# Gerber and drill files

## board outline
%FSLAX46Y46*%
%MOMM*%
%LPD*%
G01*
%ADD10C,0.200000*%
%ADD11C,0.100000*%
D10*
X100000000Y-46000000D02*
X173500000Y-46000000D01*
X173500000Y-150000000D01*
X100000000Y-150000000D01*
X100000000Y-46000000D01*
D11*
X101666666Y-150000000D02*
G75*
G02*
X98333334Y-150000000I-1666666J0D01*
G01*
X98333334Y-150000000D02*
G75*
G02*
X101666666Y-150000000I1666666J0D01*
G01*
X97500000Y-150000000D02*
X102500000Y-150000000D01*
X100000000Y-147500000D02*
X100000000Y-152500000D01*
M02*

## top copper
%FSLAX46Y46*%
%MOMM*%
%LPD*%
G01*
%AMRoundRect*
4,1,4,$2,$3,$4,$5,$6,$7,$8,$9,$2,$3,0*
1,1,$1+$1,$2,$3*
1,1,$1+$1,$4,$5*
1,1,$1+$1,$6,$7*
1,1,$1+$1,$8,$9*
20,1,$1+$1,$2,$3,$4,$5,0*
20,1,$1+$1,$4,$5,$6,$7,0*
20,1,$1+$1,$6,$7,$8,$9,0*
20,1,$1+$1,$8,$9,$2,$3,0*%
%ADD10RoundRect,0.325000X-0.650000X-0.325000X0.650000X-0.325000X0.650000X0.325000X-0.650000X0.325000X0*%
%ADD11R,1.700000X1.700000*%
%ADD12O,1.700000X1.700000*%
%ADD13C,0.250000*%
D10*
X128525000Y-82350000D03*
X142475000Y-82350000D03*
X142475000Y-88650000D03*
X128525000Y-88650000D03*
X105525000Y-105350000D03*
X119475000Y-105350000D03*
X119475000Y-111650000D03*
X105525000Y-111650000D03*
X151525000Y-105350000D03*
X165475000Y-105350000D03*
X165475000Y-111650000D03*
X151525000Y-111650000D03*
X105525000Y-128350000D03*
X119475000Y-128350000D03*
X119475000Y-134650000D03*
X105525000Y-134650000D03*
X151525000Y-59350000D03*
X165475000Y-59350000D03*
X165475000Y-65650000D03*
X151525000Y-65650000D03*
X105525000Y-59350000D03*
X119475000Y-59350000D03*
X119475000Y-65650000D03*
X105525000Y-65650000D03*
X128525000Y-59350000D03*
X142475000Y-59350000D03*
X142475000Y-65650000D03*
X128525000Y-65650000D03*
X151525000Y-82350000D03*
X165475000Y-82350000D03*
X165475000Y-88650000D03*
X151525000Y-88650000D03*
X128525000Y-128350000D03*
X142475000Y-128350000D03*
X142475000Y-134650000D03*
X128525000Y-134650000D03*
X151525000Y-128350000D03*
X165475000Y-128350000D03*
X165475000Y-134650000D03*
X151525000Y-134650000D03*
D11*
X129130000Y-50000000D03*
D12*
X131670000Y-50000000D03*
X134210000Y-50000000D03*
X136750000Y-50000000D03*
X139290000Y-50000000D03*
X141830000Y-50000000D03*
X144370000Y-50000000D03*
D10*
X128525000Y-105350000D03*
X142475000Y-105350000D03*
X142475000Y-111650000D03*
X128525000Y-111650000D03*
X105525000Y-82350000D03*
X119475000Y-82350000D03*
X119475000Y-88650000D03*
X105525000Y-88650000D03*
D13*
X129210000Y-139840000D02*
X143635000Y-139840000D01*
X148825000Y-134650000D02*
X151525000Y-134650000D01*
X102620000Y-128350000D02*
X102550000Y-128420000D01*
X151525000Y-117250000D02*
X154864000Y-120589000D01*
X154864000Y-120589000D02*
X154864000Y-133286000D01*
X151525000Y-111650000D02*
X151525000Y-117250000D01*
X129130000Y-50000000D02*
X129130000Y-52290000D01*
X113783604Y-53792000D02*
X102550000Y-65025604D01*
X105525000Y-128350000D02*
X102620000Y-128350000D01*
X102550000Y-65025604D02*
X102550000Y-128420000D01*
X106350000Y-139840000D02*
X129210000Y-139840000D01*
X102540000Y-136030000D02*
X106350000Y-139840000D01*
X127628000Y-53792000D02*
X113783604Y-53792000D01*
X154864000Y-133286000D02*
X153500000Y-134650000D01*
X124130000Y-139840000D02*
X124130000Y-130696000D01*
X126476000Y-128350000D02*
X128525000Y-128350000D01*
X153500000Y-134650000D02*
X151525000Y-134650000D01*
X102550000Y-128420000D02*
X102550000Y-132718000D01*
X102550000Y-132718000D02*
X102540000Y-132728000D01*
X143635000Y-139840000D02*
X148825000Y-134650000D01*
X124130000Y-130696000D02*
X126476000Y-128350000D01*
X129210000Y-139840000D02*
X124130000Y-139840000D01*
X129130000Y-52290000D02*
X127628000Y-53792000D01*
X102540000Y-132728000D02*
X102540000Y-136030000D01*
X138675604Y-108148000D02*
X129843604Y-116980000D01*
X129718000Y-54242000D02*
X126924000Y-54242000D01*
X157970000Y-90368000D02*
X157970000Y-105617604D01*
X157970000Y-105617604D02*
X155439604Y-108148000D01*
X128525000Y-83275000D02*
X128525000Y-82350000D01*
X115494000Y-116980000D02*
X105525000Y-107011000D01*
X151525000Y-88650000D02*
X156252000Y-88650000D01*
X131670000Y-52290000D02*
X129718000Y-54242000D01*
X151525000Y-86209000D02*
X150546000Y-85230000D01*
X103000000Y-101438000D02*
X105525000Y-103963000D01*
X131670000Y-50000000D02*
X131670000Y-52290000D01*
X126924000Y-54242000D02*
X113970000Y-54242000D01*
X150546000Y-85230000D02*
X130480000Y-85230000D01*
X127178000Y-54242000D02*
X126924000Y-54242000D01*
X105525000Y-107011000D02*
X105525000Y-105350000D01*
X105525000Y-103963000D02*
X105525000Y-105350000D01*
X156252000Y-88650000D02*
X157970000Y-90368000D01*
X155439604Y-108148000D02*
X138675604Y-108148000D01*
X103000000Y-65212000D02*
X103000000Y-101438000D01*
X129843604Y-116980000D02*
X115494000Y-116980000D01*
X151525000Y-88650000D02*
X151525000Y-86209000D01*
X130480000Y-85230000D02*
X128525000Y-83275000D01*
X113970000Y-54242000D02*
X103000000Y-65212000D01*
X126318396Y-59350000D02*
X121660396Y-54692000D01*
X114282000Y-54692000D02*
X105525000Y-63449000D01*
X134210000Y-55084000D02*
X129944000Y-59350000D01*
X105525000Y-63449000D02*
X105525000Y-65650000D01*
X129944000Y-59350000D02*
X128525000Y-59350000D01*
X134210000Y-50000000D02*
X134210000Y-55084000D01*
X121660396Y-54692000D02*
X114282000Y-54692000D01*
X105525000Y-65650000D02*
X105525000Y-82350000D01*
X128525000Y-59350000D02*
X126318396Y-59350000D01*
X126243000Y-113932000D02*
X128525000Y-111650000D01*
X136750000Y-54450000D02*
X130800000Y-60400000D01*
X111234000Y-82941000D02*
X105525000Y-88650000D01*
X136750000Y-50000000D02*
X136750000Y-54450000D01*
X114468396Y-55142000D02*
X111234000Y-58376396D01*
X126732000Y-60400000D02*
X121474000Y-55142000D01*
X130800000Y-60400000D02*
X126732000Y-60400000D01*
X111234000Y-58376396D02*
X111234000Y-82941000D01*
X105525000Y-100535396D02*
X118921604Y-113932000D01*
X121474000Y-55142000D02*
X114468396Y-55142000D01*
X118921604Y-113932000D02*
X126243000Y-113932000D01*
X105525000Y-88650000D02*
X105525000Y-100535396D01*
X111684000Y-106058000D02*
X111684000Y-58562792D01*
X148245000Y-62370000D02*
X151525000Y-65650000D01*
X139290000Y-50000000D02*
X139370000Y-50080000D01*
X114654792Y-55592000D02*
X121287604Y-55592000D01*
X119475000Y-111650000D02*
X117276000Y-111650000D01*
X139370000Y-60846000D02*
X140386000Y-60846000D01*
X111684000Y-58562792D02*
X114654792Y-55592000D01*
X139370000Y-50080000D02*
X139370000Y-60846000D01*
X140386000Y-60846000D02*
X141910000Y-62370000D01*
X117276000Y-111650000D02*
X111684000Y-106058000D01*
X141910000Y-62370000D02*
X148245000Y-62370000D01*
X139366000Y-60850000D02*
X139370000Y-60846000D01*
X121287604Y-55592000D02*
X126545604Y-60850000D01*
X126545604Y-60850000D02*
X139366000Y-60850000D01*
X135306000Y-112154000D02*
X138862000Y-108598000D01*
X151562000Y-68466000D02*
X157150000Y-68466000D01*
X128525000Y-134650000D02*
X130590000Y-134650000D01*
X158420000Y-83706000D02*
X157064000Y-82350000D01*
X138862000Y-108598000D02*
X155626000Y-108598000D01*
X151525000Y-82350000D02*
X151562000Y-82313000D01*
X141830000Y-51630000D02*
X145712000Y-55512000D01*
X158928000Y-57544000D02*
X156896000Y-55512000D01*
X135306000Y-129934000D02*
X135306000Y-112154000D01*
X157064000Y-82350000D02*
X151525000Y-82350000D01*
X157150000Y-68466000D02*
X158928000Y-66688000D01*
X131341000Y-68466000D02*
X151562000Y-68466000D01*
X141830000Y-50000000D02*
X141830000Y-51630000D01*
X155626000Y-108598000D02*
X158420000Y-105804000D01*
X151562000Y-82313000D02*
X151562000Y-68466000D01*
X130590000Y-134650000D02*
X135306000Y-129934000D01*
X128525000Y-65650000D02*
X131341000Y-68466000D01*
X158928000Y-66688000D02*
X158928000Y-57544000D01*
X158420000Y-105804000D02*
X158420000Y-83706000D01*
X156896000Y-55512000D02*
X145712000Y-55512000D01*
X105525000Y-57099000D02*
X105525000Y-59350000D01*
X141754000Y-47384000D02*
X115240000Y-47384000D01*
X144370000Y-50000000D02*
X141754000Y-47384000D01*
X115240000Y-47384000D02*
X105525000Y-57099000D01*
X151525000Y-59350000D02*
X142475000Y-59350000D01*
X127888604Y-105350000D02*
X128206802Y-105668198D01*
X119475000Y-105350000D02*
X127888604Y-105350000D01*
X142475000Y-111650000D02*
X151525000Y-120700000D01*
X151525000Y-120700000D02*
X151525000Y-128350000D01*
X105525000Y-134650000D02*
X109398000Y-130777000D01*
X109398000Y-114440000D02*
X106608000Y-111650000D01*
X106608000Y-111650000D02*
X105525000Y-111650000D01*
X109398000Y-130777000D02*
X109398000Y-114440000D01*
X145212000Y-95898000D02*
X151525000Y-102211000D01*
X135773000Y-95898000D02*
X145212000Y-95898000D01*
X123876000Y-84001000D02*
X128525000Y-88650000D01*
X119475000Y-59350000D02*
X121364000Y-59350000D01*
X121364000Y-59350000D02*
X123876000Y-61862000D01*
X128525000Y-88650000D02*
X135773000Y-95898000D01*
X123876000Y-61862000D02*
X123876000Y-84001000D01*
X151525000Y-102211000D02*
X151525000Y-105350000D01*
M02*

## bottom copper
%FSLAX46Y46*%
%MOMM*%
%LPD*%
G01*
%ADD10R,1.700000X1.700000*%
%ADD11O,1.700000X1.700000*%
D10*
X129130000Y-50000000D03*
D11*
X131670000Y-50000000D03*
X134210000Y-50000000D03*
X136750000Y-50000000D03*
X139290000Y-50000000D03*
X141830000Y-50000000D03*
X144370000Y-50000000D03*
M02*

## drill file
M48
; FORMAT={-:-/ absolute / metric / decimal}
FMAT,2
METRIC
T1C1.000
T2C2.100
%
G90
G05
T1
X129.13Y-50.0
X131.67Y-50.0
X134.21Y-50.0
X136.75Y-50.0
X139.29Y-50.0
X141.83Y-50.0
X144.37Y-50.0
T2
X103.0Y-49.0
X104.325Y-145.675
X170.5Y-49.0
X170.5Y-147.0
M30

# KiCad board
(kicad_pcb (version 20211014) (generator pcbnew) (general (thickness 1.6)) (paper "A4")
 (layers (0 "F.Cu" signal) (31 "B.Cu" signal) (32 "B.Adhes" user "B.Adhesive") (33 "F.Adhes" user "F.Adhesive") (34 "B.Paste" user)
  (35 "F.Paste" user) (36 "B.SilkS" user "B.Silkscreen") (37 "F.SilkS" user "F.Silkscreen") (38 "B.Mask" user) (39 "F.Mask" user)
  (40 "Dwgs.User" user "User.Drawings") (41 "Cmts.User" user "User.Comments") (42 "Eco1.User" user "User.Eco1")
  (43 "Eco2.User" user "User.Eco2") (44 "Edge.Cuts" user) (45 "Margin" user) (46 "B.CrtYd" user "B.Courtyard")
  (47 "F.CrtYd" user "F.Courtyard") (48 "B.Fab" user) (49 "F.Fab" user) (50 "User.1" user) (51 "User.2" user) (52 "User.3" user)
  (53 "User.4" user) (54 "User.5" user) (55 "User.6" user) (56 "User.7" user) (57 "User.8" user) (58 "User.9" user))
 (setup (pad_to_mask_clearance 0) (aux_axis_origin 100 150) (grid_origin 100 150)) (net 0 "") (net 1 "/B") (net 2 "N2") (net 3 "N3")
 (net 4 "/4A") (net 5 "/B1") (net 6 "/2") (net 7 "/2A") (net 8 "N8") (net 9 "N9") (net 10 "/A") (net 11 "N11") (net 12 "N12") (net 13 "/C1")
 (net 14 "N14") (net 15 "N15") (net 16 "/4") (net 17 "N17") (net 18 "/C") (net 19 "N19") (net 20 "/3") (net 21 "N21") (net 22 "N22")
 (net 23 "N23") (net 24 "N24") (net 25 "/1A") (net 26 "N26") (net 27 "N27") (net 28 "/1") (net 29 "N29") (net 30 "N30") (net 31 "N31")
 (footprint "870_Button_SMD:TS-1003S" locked (layer "F.Cu") (at 135.5 85.5)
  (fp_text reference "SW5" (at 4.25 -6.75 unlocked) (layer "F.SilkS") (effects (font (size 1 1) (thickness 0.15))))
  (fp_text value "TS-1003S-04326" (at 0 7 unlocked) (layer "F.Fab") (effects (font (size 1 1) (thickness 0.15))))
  (pad "1" smd roundrect locked (at -6.975 -3.15) (size 1.95 1.3) (layers "F.Cu" "F.Paste" "F.Mask") (roundrect_rratio 0.25) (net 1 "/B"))
  (pad "2" smd roundrect locked (at 6.975 -3.15) (size 1.95 1.3) (layers "F.Cu" "F.Paste" "F.Mask") (roundrect_rratio 0.25) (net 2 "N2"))
  (pad "3" smd roundrect locked (at 6.975 3.15) (size 1.95 1.3) (layers "F.Cu" "F.Paste" "F.Mask") (roundrect_rratio 0.25) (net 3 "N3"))
  (pad "4" smd roundrect locked (at -6.975 3.15) (size 1.95 1.3) (layers "F.Cu" "F.Paste" "F.Mask") (roundrect_rratio 0.25) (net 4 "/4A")))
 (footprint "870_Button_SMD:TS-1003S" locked (layer "F.Cu") (at 112.5 108.5)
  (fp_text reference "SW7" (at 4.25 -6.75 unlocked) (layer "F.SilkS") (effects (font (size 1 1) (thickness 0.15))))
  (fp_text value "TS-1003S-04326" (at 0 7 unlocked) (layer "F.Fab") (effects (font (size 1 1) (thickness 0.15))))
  (pad "1" smd roundrect locked (at -6.975 -3.15) (size 1.95 1.3) (layers "F.Cu" "F.Paste" "F.Mask") (roundrect_rratio 0.25) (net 1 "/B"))
  (pad "2" smd roundrect locked (at 6.975 -3.15) (size 1.95 1.3) (layers "F.Cu" "F.Paste" "F.Mask") (roundrect_rratio 0.25) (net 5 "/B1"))
  (pad "3" smd roundrect locked (at 6.975 3.15) (size 1.95 1.3) (layers "F.Cu" "F.Paste" "F.Mask") (roundrect_rratio 0.25) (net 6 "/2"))
  (pad "4" smd roundrect locked (at -6.975 3.15) (size 1.95 1.3) (layers "F.Cu" "F.Paste" "F.Mask") (roundrect_rratio 0.25) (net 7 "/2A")))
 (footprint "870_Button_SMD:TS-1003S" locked (layer "F.Cu") (at 158.5 108.5)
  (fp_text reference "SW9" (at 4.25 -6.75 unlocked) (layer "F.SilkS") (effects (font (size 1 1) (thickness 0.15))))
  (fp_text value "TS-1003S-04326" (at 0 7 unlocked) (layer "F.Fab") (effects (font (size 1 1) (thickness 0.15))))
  (pad "1" smd roundrect locked (at -6.975 -3.15) (size 1.95 1.3) (layers "F.Cu" "F.Paste" "F.Mask") (roundrect_rratio 0.25) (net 4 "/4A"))
  (pad "2" smd roundrect locked (at 6.975 -3.15) (size 1.95 1.3) (layers "F.Cu" "F.Paste" "F.Mask") (roundrect_rratio 0.25) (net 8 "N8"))
  (pad "3" smd roundrect locked (at 6.975 3.15) (size 1.95 1.3) (layers "F.Cu" "F.Paste" "F.Mask") (roundrect_rratio 0.25) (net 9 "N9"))
  (pad "4" smd roundrect locked (at -6.975 3.15) (size 1.95 1.3) (layers "F.Cu" "F.Paste" "F.Mask") (roundrect_rratio 0.25) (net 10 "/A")))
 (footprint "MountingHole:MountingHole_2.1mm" (layer "F.Cu") (at 104.325 145.675)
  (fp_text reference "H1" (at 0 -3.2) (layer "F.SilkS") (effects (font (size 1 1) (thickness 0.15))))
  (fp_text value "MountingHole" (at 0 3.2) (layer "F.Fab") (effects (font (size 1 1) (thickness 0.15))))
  (pad "" np_thru_hole circle (at 0 0) (size 2.1 2.1) (drill 2.1) (layers *.Cu *.Mask)))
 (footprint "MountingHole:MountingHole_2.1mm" (layer "F.Cu") (at 170.5 147)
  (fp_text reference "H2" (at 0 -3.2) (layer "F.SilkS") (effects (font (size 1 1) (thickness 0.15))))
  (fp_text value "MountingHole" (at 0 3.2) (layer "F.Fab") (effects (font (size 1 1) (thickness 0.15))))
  (pad "" np_thru_hole circle (at 0 0) (size 2.1 2.1) (drill 2.1) (layers *.Cu *.Mask)))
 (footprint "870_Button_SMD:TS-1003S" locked (layer "F.Cu") (at 112.5 131.5)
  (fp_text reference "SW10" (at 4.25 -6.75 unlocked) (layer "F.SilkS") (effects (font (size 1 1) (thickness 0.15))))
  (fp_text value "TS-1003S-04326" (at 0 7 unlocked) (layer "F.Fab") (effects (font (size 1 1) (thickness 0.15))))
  (pad "1" smd roundrect locked (at -6.975 -3.15) (size 1.95 1.3) (layers "F.Cu" "F.Paste" "F.Mask") (roundrect_rratio 0.25) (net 10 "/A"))
  (pad "2" smd roundrect locked (at 6.975 -3.15) (size 1.95 1.3) (layers "F.Cu" "F.Paste" "F.Mask") (roundrect_rratio 0.25) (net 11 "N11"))
  (pad "3" smd roundrect locked (at 6.975 3.15) (size 1.95 1.3) (layers "F.Cu" "F.Paste" "F.Mask") (roundrect_rratio 0.25) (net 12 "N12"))
  (pad "4" smd roundrect locked (at -6.975 3.15) (size 1.95 1.3) (layers "F.Cu" "F.Paste" "F.Mask") (roundrect_rratio 0.25) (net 7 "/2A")))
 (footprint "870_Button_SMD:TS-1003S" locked (layer "F.Cu") (at 158.5 62.5)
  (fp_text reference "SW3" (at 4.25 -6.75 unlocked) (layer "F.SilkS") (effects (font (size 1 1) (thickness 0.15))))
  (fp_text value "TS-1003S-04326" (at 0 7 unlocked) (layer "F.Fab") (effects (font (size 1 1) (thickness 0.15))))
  (pad "1" smd roundrect locked (at -6.975 -3.15) (size 1.95 1.3) (layers "F.Cu" "F.Paste" "F.Mask") (roundrect_rratio 0.25) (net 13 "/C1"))
  (pad "2" smd roundrect locked (at 6.975 -3.15) (size 1.95 1.3) (layers "F.Cu" "F.Paste" "F.Mask") (roundrect_rratio 0.25) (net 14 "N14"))
  (pad "3" smd roundrect locked (at 6.975 3.15) (size 1.95 1.3) (layers "F.Cu" "F.Paste" "F.Mask") (roundrect_rratio 0.25) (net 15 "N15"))
  (pad "4" smd roundrect locked (at -6.975 3.15) (size 1.95 1.3) (layers "F.Cu" "F.Paste" "F.Mask") (roundrect_rratio 0.25) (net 6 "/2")))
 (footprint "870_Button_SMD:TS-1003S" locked (layer "F.Cu") (at 112.5 62.5)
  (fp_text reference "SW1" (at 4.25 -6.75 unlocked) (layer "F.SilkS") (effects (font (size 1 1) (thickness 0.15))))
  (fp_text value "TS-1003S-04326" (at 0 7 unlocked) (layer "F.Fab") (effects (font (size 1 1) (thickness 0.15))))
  (pad "1" smd roundrect locked (at -6.975 -3.15) (size 1.95 1.3) (layers "F.Cu" "F.Paste" "F.Mask") (roundrect_rratio 0.25) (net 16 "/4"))
  (pad "2" smd roundrect locked (at 6.975 -3.15) (size 1.95 1.3) (layers "F.Cu" "F.Paste" "F.Mask") (roundrect_rratio 0.25) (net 4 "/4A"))
  (pad "3" smd roundrect locked (at 6.975 3.15) (size 1.95 1.3) (layers "F.Cu" "F.Paste" "F.Mask") (roundrect_rratio 0.25) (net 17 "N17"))
  (pad "4" smd roundrect locked (at -6.975 3.15) (size 1.95 1.3) (layers "F.Cu" "F.Paste" "F.Mask") (roundrect_rratio 0.25) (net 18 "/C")))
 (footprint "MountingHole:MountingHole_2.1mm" (layer "F.Cu") (at 103 49)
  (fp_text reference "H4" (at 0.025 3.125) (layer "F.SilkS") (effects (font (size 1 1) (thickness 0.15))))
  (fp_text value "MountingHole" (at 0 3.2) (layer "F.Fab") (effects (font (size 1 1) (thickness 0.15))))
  (pad "" np_thru_hole circle (at 0 0) (size 2.1 2.1) (drill 2.1) (layers *.Cu *.Mask)))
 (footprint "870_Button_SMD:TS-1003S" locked (layer "F.Cu") (at 135.5 62.5)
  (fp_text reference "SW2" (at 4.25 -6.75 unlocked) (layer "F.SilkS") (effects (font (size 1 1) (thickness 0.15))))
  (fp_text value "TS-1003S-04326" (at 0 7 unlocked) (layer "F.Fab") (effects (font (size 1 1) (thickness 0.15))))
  (pad "1" smd roundrect locked (at -6.975 -3.15) (size 1.95 1.3) (layers "F.Cu" "F.Paste" "F.Mask") (roundrect_rratio 0.25) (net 18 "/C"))
  (pad "2" smd roundrect locked (at 6.975 -3.15) (size 1.95 1.3) (layers "F.Cu" "F.Paste" "F.Mask") (roundrect_rratio 0.25) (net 13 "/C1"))
  (pad "3" smd roundrect locked (at 6.975 3.15) (size 1.95 1.3) (layers "F.Cu" "F.Paste" "F.Mask") (roundrect_rratio 0.25) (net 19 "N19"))
  (pad "4" smd roundrect locked (at -6.975 3.15) (size 1.95 1.3) (layers "F.Cu" "F.Paste" "F.Mask") (roundrect_rratio 0.25) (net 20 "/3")))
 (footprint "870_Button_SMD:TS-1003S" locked (layer "F.Cu") (at 158.5 85.5)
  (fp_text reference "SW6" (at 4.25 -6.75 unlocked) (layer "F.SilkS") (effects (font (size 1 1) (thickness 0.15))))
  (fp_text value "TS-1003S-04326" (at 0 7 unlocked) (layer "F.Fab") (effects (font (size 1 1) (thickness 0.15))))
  (pad "1" smd roundrect locked (at -6.975 -3.15) (size 1.95 1.3) (layers "F.Cu" "F.Paste" "F.Mask") (roundrect_rratio 0.25) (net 20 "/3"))
  (pad "2" smd roundrect locked (at 6.975 -3.15) (size 1.95 1.3) (layers "F.Cu" "F.Paste" "F.Mask") (roundrect_rratio 0.25) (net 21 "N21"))
  (pad "3" smd roundrect locked (at 6.975 3.15) (size 1.95 1.3) (layers "F.Cu" "F.Paste" "F.Mask") (roundrect_rratio 0.25) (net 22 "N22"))
  (pad "4" smd roundrect locked (at -6.975 3.15) (size 1.95 1.3) (layers "F.Cu" "F.Paste" "F.Mask") (roundrect_rratio 0.25) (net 1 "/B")))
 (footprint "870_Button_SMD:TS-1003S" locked (layer "F.Cu") (at 135.5 131.5)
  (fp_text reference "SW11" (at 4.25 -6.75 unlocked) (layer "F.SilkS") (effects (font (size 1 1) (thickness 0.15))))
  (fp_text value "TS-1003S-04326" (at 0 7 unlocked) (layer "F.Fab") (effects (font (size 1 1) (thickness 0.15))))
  (pad "1" smd roundrect locked (at -6.975 -3.15) (size 1.95 1.3) (layers "F.Cu" "F.Paste" "F.Mask") (roundrect_rratio 0.25) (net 10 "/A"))
  (pad "2" smd roundrect locked (at 6.975 -3.15) (size 1.95 1.3) (layers "F.Cu" "F.Paste" "F.Mask") (roundrect_rratio 0.25) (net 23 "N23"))
  (pad "3" smd roundrect locked (at 6.975 3.15) (size 1.95 1.3) (layers "F.Cu" "F.Paste" "F.Mask") (roundrect_rratio 0.25) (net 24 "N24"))
  (pad "4" smd roundrect locked (at -6.975 3.15) (size 1.95 1.3) (layers "F.Cu" "F.Paste" "F.Mask") (roundrect_rratio 0.25) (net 20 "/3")))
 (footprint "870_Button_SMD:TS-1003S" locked (layer "F.Cu") (at 158.5 131.5)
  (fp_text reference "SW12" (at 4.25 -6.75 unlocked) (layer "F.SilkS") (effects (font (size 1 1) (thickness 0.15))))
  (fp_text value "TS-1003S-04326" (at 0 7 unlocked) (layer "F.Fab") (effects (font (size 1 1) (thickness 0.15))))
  (pad "1" smd roundrect locked (at -6.975 -3.15) (size 1.95 1.3) (layers "F.Cu" "F.Paste" "F.Mask") (roundrect_rratio 0.25) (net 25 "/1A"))
  (pad "2" smd roundrect locked (at 6.975 -3.15) (size 1.95 1.3) (layers "F.Cu" "F.Paste" "F.Mask") (roundrect_rratio 0.25) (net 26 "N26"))
  (pad "3" smd roundrect locked (at 6.975 3.15) (size 1.95 1.3) (layers "F.Cu" "F.Paste" "F.Mask") (roundrect_rratio 0.25) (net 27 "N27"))
  (pad "4" smd roundrect locked (at -6.975 3.15) (size 1.95 1.3) (layers "F.Cu" "F.Paste" "F.Mask") (roundrect_rratio 0.25) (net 10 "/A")))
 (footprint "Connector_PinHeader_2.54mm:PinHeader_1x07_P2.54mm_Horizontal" (layer "F.Cu") (at 129.13 50 90)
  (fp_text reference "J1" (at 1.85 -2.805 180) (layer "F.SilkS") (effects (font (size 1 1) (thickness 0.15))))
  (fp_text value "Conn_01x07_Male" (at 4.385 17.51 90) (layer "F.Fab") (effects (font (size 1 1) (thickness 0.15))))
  (pad "1" thru_hole rect (at 0 0 90) (size 1.7 1.7) (drill 1) (layers *.Cu *.Mask) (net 10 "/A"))
  (pad "2" thru_hole oval (at 0 2.54 90) (size 1.7 1.7) (drill 1) (layers *.Cu *.Mask) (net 1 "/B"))
  (pad "3" thru_hole oval (at 0 5.08 90) (size 1.7 1.7) (drill 1) (layers *.Cu *.Mask) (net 18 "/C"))
  (pad "4" thru_hole oval (at 0 7.62 90) (size 1.7 1.7) (drill 1) (layers *.Cu *.Mask) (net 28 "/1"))
  (pad "5" thru_hole oval (at 0 10.16 90) (size 1.7 1.7) (drill 1) (layers *.Cu *.Mask) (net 6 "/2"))
  (pad "6" thru_hole oval (at 0 12.7 90) (size 1.7 1.7) (drill 1) (layers *.Cu *.Mask) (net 20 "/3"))
  (pad "7" thru_hole oval (at 0 15.24 90) (size 1.7 1.7) (drill 1) (layers *.Cu *.Mask) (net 16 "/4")))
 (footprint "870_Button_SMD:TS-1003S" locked (layer "F.Cu") (at 135.5 108.5)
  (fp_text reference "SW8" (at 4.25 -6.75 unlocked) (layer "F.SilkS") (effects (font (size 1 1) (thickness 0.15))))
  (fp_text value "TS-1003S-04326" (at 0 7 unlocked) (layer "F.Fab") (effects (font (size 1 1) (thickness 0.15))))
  (pad "1" smd roundrect locked (at -6.975 -3.15) (size 1.95 1.3) (layers "F.Cu" "F.Paste" "F.Mask") (roundrect_rratio 0.25) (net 5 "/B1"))
  (pad "2" smd roundrect locked (at 6.975 -3.15) (size 1.95 1.3) (layers "F.Cu" "F.Paste" "F.Mask") (roundrect_rratio 0.25) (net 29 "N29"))
  (pad "3" smd roundrect locked (at 6.975 3.15) (size 1.95 1.3) (layers "F.Cu" "F.Paste" "F.Mask") (roundrect_rratio 0.25) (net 25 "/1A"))
  (pad "4" smd roundrect locked (at -6.975 3.15) (size 1.95 1.3) (layers "F.Cu" "F.Paste" "F.Mask") (roundrect_rratio 0.25) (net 28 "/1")))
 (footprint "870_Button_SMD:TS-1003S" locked (layer "F.Cu") (at 112.5 85.5)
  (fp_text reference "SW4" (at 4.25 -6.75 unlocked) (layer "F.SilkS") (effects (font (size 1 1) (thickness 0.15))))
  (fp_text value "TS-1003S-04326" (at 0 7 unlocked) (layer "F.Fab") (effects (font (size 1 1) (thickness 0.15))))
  (pad "1" smd roundrect locked (at -6.975 -3.15) (size 1.95 1.3) (layers "F.Cu" "F.Paste" "F.Mask") (roundrect_rratio 0.25) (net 18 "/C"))
  (pad "2" smd roundrect locked (at 6.975 -3.15) (size 1.95 1.3) (layers "F.Cu" "F.Paste" "F.Mask") (roundrect_rratio 0.25) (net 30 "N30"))
  (pad "3" smd roundrect locked (at 6.975 3.15) (size 1.95 1.3) (layers "F.Cu" "F.Paste" "F.Mask") (roundrect_rratio 0.25) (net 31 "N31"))
  (pad "4" smd roundrect locked (at -6.975 3.15) (size 1.95 1.3) (layers "F.Cu" "F.Paste" "F.Mask") (roundrect_rratio 0.25) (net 28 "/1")))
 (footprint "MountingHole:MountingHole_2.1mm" (layer "F.Cu") (at 170.5 49)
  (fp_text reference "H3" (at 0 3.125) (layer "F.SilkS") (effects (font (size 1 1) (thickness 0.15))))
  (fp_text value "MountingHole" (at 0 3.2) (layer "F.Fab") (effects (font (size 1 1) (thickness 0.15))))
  (pad "" np_thru_hole circle (at 0 0) (size 2.1 2.1) (drill 2.1) (layers *.Cu *.Mask)))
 (gr_rect (start 100 150) (end 173.5 46) (layer "Edge.Cuts") (width 0.2) (fill none))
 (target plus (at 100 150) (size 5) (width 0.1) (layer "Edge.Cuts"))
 (segment (start 129.21 139.84) (end 143.635 139.84) (width 0.25) (layer "F.Cu") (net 10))
 (segment (start 148.825 134.65) (end 151.525 134.65) (width 0.25) (layer "F.Cu") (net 10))
 (segment (start 102.62 128.35) (end 102.55 128.42) (width 0.25) (layer "F.Cu") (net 10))
 (segment (start 151.525 117.25) (end 154.864 120.589) (width 0.25) (layer "F.Cu") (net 10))
 (segment (start 154.864 120.589) (end 154.864 133.286) (width 0.25) (layer "F.Cu") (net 10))
 (segment (start 151.525 111.65) (end 151.525 117.25) (width 0.25) (layer "F.Cu") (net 10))
 (segment (start 129.13 50) (end 129.13 52.29) (width 0.25) (layer "F.Cu") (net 10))
 (segment (start 113.783604 53.792) (end 102.55 65.025604) (width 0.25) (layer "F.Cu") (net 10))
 (segment (start 105.525 128.35) (end 102.62 128.35) (width 0.25) (layer "F.Cu") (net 10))
 (segment (start 102.55 65.025604) (end 102.55 128.42) (width 0.25) (layer "F.Cu") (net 10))
 (segment (start 106.35 139.84) (end 129.21 139.84) (width 0.25) (layer "F.Cu") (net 10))
 (segment (start 102.54 136.03) (end 106.35 139.84) (width 0.25) (layer "F.Cu") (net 10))
 (segment (start 127.628 53.792) (end 113.783604 53.792) (width 0.25) (layer "F.Cu") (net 10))
 (segment (start 154.864 133.286) (end 153.5 134.65) (width 0.25) (layer "F.Cu") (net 10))
 (segment (start 124.13 139.84) (end 124.13 130.696) (width 0.25) (layer "F.Cu") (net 10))
 (segment (start 126.476 128.35) (end 128.525 128.35) (width 0.25) (layer "F.Cu") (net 10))
 (segment (start 153.5 134.65) (end 151.525 134.65) (width 0.25) (layer "F.Cu") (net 10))
 (segment (start 102.55 128.42) (end 102.55 132.718) (width 0.25) (layer "F.Cu") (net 10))
 (segment (start 102.55 132.718) (end 102.54 132.728) (width 0.25) (layer "F.Cu") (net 10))
 (segment (start 143.635 139.84) (end 148.825 134.65) (width 0.25) (layer "F.Cu") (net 10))
 (segment (start 124.13 130.696) (end 126.476 128.35) (width 0.25) (layer "F.Cu") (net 10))
 (segment (start 129.21 139.84) (end 124.13 139.84) (width 0.25) (layer "F.Cu") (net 10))
 (segment (start 129.13 52.29) (end 127.628 53.792) (width 0.25) (layer "F.Cu") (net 10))
 (segment (start 102.54 132.728) (end 102.54 136.03) (width 0.25) (layer "F.Cu") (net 10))
 (segment (start 138.675604 108.148) (end 129.843604 116.98) (width 0.25) (layer "F.Cu") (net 1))
 (segment (start 129.718 54.242) (end 126.924 54.242) (width 0.25) (layer "F.Cu") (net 1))
 (segment (start 157.97 90.368) (end 157.97 105.617604) (width 0.25) (layer "F.Cu") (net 1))
 (segment (start 157.97 105.617604) (end 155.439604 108.148) (width 0.25) (layer "F.Cu") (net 1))
 (segment (start 128.525 83.275) (end 128.525 82.35) (width 0.25) (layer "F.Cu") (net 1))
 (segment (start 115.494 116.98) (end 105.525 107.011) (width 0.25) (layer "F.Cu") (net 1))
 (segment (start 151.525 88.65) (end 156.252 88.65) (width 0.25) (layer "F.Cu") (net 1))
 (segment (start 131.67 52.29) (end 129.718 54.242) (width 0.25) (layer "F.Cu") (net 1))
 (segment (start 151.525 86.209) (end 150.546 85.23) (width 0.25) (layer "F.Cu") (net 1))
 (segment (start 103 101.438) (end 105.525 103.963) (width 0.25) (layer "F.Cu") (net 1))
 (segment (start 131.67 50) (end 131.67 52.29) (width 0.25) (layer "F.Cu") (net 1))
 (segment (start 126.924 54.242) (end 113.97 54.242) (width 0.25) (layer "F.Cu") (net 1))
 (segment (start 150.546 85.23) (end 130.48 85.23) (width 0.25) (layer "F.Cu") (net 1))
 (segment (start 127.178 54.242) (end 126.924 54.242) (width 0.25) (layer "F.Cu") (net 1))
 (segment (start 105.525 107.011) (end 105.525 105.35) (width 0.25) (layer "F.Cu") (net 1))
 (segment (start 105.525 103.963) (end 105.525 105.35) (width 0.25) (layer "F.Cu") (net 1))
 (segment (start 156.252 88.65) (end 157.97 90.368) (width 0.25) (layer "F.Cu") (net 1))
 (segment (start 155.439604 108.148) (end 138.675604 108.148) (width 0.25) (layer "F.Cu") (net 1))
 (segment (start 103 65.212) (end 103 101.438) (width 0.25) (layer "F.Cu") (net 1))
 (segment (start 129.843604 116.98) (end 115.494 116.98) (width 0.25) (layer "F.Cu") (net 1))
 (segment (start 151.525 88.65) (end 151.525 86.209) (width 0.25) (layer "F.Cu") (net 1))
 (segment (start 130.48 85.23) (end 128.525 83.275) (width 0.25) (layer "F.Cu") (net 1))
 (segment (start 113.97 54.242) (end 103 65.212) (width 0.25) (layer "F.Cu") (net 1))
 (segment (start 126.318396 59.35) (end 121.660396 54.692) (width 0.25) (layer "F.Cu") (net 18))
 (segment (start 114.282 54.692) (end 105.525 63.449) (width 0.25) (layer "F.Cu") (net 18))
 (segment (start 134.21 55.084) (end 129.944 59.35) (width 0.25) (layer "F.Cu") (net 18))
 (segment (start 105.525 63.449) (end 105.525 65.65) (width 0.25) (layer "F.Cu") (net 18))
 (segment (start 129.944 59.35) (end 128.525 59.35) (width 0.25) (layer "F.Cu") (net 18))
 (segment (start 134.21 50) (end 134.21 55.084) (width 0.25) (layer "F.Cu") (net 18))
 (segment (start 121.660396 54.692) (end 114.282 54.692) (width 0.25) (layer "F.Cu") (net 18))
 (segment (start 105.525 65.65) (end 105.525 82.35) (width 0.25) (layer "F.Cu") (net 18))
 (segment (start 128.525 59.35) (end 126.318396 59.35) (width 0.25) (layer "F.Cu") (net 18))
 (segment (start 126.243 113.932) (end 128.525 111.65) (width 0.25) (layer "F.Cu") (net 28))
 (segment (start 136.75 54.45) (end 130.8 60.4) (width 0.25) (layer "F.Cu") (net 28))
 (segment (start 111.234 82.941) (end 105.525 88.65) (width 0.25) (layer "F.Cu") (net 28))
 (segment (start 136.75 50) (end 136.75 54.45) (width 0.25) (layer "F.Cu") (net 28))
 (segment (start 114.468396 55.142) (end 111.234 58.376396) (width 0.25) (layer "F.Cu") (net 28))
 (segment (start 126.732 60.4) (end 121.474 55.142) (width 0.25) (layer "F.Cu") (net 28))
 (segment (start 130.8 60.4) (end 126.732 60.4) (width 0.25) (layer "F.Cu") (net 28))
 (segment (start 111.234 58.376396) (end 111.234 82.941) (width 0.25) (layer "F.Cu") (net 28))
 (segment (start 105.525 100.535396) (end 118.921604 113.932) (width 0.25) (layer "F.Cu") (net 28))
 (segment (start 121.474 55.142) (end 114.468396 55.142) (width 0.25) (layer "F.Cu") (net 28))
 (segment (start 118.921604 113.932) (end 126.243 113.932) (width 0.25) (layer "F.Cu") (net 28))
 (segment (start 105.525 88.65) (end 105.525 100.535396) (width 0.25) (layer "F.Cu") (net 28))
 (segment (start 111.684 106.058) (end 111.684 58.562792) (width 0.25) (layer "F.Cu") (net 6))
 (segment (start 148.245 62.37) (end 151.525 65.65) (width 0.25) (layer "F.Cu") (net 6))
 (segment (start 139.29 50) (end 139.37 50.08) (width 0.25) (layer "F.Cu") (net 6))
 (segment (start 114.654792 55.592) (end 121.287604 55.592) (width 0.25) (layer "F.Cu") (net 6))
 (segment (start 119.475 111.65) (end 117.276 111.65) (width 0.25) (layer "F.Cu") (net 6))
 (segment (start 139.37 60.846) (end 140.386 60.846) (width 0.25) (layer "F.Cu") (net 6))
 (segment (start 111.684 58.562792) (end 114.654792 55.592) (width 0.25) (layer "F.Cu") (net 6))
 (segment (start 139.37 50.08) (end 139.37 60.846) (width 0.25) (layer "F.Cu") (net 6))
 (segment (start 140.386 60.846) (end 141.91 62.37) (width 0.25) (layer "F.Cu") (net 6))
 (segment (start 117.276 111.65) (end 111.684 106.058) (width 0.25) (layer "F.Cu") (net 6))
 (segment (start 141.91 62.37) (end 148.245 62.37) (width 0.25) (layer "F.Cu") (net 6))
 (segment (start 139.366 60.85) (end 139.37 60.846) (width 0.25) (layer "F.Cu") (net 6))
 (segment (start 121.287604 55.592) (end 126.545604 60.85) (width 0.25) (layer "F.Cu") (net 6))
 (segment (start 126.545604 60.85) (end 139.366 60.85) (width 0.25) (layer "F.Cu") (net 6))
 (segment (start 135.306 112.154) (end 138.862 108.598) (width 0.25) (layer "F.Cu") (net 20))
 (segment (start 151.562 68.466) (end 157.15 68.466) (width 0.25) (layer "F.Cu") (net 20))
 (segment (start 128.525 134.65) (end 130.59 134.65) (width 0.25) (layer "F.Cu") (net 20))
 (segment (start 158.42 83.706) (end 157.064 82.35) (width 0.25) (layer "F.Cu") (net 20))
 (segment (start 138.862 108.598) (end 155.626 108.598) (width 0.25) (layer "F.Cu") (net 20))
 (segment (start 151.525 82.35) (end 151.562 82.313) (width 0.25) (layer "F.Cu") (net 20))
 (segment (start 141.83 51.63) (end 145.712 55.512) (width 0.25) (layer "F.Cu") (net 20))
 (segment (start 158.928 57.544) (end 156.896 55.512) (width 0.25) (layer "F.Cu") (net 20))
 (segment (start 135.306 129.934) (end 135.306 112.154) (width 0.25) (layer "F.Cu") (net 20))
 (segment (start 157.064 82.35) (end 151.525 82.35) (width 0.25) (layer "F.Cu") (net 20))
 (segment (start 157.15 68.466) (end 158.928 66.688) (width 0.25) (layer "F.Cu") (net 20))
 (segment (start 131.341 68.466) (end 151.562 68.466) (width 0.25) (layer "F.Cu") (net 20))
 (segment (start 141.83 50) (end 141.83 51.63) (width 0.25) (layer "F.Cu") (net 20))
 (segment (start 155.626 108.598) (end 158.42 105.804) (width 0.25) (layer "F.Cu") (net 20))
 (segment (start 151.562 82.313) (end 151.562 68.466) (width 0.25) (layer "F.Cu") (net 20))
 (segment (start 130.59 134.65) (end 135.306 129.934) (width 0.25) (layer "F.Cu") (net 20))
 (segment (start 128.525 65.65) (end 131.341 68.466) (width 0.25) (layer "F.Cu") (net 20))
 (segment (start 158.928 66.688) (end 158.928 57.544) (width 0.25) (layer "F.Cu") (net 20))
 (segment (start 158.42 105.804) (end 158.42 83.706) (width 0.25) (layer "F.Cu") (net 20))
 (segment (start 156.896 55.512) (end 145.712 55.512) (width 0.25) (layer "F.Cu") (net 20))
 (segment (start 105.525 57.099) (end 105.525 59.35) (width 0.25) (layer "F.Cu") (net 16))
 (segment (start 141.754 47.384) (end 115.24 47.384) (width 0.25) (layer "F.Cu") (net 16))
 (segment (start 144.37 50) (end 141.754 47.384) (width 0.25) (layer "F.Cu") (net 16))
 (segment (start 115.24 47.384) (end 105.525 57.099) (width 0.25) (layer "F.Cu") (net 16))
 (segment (start 151.525 59.35) (end 142.475 59.35) (width 0.25) (layer "F.Cu") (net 13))
 (segment (start 127.888604 105.35) (end 128.206802 105.668198) (width 0.25) (layer "F.Cu") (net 5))
 (segment (start 119.475 105.35) (end 127.888604 105.35) (width 0.25) (layer "F.Cu") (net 5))
 (segment (start 142.475 111.65) (end 151.525 120.7) (width 0.25) (layer "F.Cu") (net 25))
 (segment (start 151.525 120.7) (end 151.525 128.35) (width 0.25) (layer "F.Cu") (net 25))
 (segment (start 105.525 134.65) (end 109.398 130.777) (width 0.25) (layer "F.Cu") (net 7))
 (segment (start 109.398 114.44) (end 106.608 111.65) (width 0.25) (layer "F.Cu") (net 7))
 (segment (start 106.608 111.65) (end 105.525 111.65) (width 0.25) (layer "F.Cu") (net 7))
 (segment (start 109.398 130.777) (end 109.398 114.44) (width 0.25) (layer "F.Cu") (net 7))
 (segment (start 145.212 95.898) (end 151.525 102.211) (width 0.25) (layer "F.Cu") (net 4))
 (segment (start 135.773 95.898) (end 145.212 95.898) (width 0.25) (layer "F.Cu") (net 4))
 (segment (start 123.876 84.001) (end 128.525 88.65) (width 0.25) (layer "F.Cu") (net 4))
 (segment (start 119.475 59.35) (end 121.364 59.35) (width 0.25) (layer "F.Cu") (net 4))
 (segment (start 121.364 59.35) (end 123.876 61.862) (width 0.25) (layer "F.Cu") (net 4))
 (segment (start 128.525 88.65) (end 135.773 95.898) (width 0.25) (layer "F.Cu") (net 4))
 (segment (start 123.876 61.862) (end 123.876 84.001) (width 0.25) (layer "F.Cu") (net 4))
 (segment (start 151.525 102.211) (end 151.525 105.35) (width 0.25) (layer "F.Cu") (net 4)))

